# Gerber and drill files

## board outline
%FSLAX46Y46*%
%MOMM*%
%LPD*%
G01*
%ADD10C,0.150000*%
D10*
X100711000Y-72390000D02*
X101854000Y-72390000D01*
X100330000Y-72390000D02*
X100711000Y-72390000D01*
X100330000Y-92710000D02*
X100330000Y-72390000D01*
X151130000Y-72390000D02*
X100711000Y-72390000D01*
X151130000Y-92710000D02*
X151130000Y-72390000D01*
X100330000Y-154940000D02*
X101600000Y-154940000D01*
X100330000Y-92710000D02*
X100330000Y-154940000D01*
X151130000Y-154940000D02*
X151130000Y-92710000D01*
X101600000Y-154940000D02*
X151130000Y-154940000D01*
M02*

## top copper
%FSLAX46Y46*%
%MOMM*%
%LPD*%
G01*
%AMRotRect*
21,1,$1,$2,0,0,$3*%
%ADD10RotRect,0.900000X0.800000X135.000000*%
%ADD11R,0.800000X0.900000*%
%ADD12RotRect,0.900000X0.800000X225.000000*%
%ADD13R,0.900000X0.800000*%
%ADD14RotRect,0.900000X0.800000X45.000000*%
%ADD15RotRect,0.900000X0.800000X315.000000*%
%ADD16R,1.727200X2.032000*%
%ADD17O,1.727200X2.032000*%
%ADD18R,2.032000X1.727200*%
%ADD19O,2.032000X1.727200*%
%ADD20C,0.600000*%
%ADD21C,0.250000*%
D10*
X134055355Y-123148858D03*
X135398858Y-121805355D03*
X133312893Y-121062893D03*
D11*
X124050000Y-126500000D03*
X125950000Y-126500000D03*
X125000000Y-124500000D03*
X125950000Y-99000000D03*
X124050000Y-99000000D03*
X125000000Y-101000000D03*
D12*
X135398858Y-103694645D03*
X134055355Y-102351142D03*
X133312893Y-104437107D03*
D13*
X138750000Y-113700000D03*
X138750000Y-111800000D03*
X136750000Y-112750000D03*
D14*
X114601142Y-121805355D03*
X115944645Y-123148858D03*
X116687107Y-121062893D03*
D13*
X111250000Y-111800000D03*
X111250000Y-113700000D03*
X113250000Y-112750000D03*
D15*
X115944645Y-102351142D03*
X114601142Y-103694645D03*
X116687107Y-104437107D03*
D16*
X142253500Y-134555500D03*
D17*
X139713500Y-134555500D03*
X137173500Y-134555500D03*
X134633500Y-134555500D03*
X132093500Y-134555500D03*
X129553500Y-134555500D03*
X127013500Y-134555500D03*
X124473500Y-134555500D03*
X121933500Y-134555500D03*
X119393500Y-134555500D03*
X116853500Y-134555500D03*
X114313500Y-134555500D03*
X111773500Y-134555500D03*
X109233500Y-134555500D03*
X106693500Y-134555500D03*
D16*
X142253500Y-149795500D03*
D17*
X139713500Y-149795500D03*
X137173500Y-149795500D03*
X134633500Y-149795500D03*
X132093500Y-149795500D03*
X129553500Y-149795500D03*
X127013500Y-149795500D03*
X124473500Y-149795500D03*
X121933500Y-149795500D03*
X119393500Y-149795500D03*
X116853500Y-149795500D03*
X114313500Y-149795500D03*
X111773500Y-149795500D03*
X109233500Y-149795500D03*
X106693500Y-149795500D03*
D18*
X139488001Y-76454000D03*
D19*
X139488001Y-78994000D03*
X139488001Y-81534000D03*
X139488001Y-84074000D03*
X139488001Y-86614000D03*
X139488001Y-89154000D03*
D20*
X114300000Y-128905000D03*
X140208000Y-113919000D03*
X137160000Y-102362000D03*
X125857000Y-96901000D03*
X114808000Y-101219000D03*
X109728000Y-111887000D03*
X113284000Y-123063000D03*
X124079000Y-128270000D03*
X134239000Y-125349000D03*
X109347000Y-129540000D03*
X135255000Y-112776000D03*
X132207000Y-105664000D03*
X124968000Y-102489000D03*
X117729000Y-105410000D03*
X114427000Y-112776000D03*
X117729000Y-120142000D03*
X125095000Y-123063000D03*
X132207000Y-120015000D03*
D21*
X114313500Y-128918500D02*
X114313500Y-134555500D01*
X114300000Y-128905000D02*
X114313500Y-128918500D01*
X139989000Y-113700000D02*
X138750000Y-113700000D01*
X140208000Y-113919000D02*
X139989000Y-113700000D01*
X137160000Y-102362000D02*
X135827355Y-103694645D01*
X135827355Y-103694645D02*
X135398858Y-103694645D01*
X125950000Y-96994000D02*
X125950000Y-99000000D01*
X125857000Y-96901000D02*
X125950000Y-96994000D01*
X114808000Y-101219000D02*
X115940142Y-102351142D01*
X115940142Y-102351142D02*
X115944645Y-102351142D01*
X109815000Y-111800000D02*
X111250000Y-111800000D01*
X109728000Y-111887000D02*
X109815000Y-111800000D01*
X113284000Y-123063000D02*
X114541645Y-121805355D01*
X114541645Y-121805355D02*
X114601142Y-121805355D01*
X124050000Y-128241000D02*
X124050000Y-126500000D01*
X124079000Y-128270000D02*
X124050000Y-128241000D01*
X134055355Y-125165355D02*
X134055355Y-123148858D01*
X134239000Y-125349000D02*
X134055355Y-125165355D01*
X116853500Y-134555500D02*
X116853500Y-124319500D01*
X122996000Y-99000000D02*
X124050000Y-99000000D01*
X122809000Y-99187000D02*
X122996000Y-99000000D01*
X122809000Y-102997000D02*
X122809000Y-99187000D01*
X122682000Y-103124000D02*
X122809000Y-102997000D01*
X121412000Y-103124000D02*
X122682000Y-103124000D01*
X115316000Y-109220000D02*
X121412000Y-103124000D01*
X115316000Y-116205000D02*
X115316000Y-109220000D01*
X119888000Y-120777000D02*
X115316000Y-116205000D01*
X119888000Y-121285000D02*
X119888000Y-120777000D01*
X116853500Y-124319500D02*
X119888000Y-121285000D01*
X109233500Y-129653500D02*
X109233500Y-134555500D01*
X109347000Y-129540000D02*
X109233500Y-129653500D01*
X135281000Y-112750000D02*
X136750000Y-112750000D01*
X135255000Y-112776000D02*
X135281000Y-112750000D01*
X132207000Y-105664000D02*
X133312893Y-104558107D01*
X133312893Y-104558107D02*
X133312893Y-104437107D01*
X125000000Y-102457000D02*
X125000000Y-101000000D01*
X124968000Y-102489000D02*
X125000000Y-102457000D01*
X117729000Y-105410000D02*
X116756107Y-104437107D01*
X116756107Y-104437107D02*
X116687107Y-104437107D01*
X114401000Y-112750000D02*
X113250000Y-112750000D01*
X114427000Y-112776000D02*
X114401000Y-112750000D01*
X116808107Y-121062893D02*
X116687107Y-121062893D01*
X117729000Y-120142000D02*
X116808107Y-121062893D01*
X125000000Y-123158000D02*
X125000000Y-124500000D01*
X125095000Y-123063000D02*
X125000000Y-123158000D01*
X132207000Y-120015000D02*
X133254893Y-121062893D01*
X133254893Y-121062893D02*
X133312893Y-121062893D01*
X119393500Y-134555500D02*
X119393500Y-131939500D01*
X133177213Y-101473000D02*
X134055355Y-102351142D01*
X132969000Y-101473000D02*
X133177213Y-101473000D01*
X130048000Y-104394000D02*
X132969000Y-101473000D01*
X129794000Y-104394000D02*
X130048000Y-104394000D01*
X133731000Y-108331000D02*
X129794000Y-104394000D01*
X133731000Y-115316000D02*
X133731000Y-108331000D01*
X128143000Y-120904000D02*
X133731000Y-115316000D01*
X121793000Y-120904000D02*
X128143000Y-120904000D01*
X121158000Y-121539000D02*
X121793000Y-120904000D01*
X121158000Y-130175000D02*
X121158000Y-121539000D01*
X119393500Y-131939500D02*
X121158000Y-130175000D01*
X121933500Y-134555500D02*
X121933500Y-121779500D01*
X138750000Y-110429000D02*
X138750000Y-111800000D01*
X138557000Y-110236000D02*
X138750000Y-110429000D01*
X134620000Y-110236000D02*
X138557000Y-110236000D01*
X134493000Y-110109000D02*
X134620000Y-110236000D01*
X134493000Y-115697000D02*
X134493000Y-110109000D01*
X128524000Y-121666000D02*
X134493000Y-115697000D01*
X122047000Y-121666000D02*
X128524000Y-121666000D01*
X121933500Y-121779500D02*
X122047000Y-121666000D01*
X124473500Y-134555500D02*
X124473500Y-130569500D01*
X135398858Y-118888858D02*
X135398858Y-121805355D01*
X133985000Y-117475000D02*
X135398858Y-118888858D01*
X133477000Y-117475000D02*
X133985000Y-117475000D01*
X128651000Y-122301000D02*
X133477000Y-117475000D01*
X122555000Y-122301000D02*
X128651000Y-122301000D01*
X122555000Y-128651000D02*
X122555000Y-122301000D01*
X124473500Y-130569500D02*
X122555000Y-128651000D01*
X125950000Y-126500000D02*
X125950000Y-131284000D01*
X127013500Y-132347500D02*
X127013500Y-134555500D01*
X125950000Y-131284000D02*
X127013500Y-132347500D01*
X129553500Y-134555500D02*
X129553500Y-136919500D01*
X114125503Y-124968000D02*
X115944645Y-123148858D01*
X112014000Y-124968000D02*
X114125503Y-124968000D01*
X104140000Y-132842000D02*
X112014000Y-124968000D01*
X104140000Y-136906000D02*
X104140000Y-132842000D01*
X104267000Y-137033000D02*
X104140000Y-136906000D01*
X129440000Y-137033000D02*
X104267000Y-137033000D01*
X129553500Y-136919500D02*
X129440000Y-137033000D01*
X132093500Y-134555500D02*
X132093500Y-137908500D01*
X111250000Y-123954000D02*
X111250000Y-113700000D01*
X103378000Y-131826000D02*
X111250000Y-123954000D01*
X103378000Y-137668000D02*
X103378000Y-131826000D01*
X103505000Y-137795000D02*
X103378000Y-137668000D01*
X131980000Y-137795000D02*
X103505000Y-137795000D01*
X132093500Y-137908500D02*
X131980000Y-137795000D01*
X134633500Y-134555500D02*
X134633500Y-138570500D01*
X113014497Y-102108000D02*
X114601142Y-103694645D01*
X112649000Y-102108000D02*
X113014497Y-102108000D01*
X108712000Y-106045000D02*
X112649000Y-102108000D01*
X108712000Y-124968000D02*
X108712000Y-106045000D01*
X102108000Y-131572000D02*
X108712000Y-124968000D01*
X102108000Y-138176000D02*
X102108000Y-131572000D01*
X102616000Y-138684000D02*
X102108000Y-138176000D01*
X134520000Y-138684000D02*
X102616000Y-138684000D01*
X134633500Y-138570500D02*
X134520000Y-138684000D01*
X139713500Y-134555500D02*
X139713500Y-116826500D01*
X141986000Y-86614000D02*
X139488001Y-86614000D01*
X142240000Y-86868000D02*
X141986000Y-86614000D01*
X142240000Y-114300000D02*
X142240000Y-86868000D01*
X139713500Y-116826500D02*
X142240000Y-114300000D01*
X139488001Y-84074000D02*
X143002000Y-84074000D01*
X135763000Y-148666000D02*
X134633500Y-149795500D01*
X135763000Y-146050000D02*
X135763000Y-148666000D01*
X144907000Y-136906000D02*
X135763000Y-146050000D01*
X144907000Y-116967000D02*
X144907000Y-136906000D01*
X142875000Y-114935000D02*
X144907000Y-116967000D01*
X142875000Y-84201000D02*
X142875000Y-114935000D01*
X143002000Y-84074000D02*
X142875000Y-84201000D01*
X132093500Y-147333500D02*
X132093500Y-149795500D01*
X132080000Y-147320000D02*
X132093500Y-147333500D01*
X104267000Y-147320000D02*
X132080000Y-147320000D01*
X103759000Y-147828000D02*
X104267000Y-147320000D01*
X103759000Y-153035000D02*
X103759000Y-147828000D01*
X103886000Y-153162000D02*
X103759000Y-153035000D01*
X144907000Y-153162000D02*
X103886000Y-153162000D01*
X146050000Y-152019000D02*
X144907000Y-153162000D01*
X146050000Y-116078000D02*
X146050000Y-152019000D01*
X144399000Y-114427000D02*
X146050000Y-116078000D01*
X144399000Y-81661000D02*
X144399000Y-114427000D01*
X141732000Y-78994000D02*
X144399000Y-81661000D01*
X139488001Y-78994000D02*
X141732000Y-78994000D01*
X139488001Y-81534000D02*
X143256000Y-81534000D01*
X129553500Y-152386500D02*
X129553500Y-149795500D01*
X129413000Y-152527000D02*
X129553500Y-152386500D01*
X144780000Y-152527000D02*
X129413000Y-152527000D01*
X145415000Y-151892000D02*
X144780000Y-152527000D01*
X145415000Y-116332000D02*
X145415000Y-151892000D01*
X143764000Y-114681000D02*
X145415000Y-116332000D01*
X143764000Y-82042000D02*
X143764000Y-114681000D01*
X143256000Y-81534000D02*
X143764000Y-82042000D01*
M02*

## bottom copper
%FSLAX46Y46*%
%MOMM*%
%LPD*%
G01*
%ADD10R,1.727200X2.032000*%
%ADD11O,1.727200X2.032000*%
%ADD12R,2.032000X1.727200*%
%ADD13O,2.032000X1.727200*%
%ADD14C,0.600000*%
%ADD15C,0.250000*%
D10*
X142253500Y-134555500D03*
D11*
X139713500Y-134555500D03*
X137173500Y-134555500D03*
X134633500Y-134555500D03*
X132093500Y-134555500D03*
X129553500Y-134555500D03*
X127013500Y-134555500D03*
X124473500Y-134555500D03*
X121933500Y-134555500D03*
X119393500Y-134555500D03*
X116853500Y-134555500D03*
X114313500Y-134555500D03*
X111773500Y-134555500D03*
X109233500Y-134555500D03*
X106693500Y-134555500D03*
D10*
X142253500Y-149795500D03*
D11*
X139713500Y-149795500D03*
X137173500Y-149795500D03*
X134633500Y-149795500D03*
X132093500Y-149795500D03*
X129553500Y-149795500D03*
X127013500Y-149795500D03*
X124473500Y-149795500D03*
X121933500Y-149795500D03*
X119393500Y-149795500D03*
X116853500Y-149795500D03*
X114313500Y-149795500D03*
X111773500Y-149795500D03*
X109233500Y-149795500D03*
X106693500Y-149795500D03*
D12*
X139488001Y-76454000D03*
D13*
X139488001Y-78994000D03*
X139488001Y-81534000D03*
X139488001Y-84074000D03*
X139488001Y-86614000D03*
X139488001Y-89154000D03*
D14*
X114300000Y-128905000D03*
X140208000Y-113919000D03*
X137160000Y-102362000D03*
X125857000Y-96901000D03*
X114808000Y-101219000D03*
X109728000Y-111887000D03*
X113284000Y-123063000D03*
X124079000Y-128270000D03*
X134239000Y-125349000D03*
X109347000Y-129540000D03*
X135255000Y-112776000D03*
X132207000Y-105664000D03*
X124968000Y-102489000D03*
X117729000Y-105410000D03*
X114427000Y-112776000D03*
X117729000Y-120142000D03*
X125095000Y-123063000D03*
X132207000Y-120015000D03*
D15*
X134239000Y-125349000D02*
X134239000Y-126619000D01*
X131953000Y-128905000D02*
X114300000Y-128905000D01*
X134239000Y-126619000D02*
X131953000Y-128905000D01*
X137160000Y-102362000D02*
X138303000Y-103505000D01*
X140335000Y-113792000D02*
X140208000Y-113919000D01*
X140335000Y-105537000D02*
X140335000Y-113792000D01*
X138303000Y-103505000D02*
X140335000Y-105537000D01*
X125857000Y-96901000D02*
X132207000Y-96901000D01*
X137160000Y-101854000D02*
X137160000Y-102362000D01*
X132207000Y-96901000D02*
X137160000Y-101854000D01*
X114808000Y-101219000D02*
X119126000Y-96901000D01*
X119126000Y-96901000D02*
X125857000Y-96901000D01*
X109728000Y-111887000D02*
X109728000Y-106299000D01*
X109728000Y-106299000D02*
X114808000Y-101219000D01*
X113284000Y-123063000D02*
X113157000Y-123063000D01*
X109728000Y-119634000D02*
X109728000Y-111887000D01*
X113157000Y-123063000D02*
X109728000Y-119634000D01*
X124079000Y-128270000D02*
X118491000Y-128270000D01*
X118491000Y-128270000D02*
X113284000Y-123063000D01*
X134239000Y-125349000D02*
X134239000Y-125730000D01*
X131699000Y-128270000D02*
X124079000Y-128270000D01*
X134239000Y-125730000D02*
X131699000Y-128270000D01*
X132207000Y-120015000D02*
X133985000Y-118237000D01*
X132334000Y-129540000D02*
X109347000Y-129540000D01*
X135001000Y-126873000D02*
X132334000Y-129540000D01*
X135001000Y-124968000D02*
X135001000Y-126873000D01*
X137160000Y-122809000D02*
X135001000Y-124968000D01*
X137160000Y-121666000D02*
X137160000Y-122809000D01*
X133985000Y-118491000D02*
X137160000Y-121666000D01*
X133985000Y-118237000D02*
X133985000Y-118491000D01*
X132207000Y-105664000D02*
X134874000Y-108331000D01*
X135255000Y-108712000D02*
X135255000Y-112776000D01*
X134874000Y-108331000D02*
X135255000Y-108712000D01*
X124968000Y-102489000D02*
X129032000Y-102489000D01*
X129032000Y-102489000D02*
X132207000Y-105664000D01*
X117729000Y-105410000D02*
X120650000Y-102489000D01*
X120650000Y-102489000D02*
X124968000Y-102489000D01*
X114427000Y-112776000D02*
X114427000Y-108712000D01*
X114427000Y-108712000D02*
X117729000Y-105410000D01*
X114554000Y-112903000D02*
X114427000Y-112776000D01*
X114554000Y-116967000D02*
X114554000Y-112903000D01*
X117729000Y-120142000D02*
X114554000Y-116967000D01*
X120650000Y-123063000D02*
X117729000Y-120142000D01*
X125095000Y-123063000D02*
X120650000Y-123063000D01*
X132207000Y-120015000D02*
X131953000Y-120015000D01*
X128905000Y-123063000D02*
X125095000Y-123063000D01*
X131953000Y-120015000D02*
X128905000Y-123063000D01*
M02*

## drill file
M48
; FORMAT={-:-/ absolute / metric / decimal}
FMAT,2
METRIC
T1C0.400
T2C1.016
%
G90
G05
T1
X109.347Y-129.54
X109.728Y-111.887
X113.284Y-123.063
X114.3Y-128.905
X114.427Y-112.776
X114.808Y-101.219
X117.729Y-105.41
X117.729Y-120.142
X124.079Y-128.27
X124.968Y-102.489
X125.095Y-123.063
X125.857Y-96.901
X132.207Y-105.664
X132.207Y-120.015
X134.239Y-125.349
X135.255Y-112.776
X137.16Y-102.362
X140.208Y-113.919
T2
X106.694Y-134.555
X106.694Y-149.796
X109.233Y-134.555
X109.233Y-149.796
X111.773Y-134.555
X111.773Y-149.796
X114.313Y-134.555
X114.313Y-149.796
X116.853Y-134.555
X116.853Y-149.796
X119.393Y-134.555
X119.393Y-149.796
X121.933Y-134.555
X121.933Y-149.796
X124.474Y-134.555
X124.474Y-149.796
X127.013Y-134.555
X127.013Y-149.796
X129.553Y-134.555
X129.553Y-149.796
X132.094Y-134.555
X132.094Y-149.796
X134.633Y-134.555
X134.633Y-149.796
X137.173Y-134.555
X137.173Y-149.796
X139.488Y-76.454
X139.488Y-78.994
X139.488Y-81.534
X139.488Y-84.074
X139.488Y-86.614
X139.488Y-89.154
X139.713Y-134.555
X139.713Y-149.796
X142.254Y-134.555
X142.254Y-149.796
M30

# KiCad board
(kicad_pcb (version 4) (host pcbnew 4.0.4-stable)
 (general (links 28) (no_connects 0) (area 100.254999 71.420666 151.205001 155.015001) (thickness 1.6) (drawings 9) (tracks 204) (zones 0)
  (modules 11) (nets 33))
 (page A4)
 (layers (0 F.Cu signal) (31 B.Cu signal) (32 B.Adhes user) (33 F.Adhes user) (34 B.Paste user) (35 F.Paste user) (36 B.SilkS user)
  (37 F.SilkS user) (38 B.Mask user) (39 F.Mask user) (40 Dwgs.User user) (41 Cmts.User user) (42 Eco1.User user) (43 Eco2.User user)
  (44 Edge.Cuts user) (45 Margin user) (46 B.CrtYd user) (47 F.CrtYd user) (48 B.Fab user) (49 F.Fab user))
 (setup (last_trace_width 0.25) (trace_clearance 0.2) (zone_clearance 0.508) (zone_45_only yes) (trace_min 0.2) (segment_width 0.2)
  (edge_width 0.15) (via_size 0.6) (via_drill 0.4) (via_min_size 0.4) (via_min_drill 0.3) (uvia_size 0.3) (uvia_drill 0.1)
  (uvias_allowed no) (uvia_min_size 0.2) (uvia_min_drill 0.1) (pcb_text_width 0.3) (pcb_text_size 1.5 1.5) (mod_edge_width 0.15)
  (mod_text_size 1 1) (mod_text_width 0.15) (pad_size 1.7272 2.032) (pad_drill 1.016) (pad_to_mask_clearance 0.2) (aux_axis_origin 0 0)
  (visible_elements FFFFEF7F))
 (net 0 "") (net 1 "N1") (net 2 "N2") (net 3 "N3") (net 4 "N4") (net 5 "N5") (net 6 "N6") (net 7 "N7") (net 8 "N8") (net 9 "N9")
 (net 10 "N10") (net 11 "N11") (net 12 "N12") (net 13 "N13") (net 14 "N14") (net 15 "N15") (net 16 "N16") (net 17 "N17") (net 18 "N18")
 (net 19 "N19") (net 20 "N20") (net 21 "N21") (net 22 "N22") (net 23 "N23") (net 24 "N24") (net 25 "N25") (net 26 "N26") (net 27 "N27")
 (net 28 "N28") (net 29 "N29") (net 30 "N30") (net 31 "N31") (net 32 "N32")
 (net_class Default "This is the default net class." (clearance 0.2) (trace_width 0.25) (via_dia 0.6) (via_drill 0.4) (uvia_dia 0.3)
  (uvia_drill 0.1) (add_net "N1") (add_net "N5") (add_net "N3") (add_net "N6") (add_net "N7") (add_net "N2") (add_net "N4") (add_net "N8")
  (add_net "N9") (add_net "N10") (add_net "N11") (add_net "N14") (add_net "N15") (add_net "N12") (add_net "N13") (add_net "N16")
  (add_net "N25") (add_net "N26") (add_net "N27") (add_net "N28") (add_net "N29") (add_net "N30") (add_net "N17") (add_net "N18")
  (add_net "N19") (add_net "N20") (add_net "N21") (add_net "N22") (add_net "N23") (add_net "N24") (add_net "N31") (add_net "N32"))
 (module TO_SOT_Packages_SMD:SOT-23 (layer F.Cu) (at 134.02 121.77 135)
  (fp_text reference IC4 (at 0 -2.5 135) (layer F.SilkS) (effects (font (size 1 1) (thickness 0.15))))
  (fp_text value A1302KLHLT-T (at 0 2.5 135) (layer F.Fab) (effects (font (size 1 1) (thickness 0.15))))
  (pad 1 smd rect (at -1 -0.95 135) (size 0.9 0.8) (layers F.Cu F.Paste F.Mask) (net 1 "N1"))
  (pad 2 smd rect (at -1 0.95 135) (size 0.9 0.8) (layers F.Cu F.Paste F.Mask) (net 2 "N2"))
  (pad 3 smd rect (at 1 0 135) (size 0.9 0.8) (layers F.Cu F.Paste F.Mask) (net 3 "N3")))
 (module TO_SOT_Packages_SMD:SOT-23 (layer F.Cu) (at 125 125.5 90)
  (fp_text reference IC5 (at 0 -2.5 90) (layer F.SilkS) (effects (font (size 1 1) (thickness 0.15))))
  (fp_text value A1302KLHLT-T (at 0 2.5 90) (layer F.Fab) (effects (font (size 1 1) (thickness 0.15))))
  (pad 1 smd rect (at -1 -0.95 90) (size 0.9 0.8) (layers F.Cu F.Paste F.Mask) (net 1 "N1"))
  (pad 2 smd rect (at -1 0.95 90) (size 0.9 0.8) (layers F.Cu F.Paste F.Mask) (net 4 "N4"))
  (pad 3 smd rect (at 1 0 90) (size 0.9 0.8) (layers F.Cu F.Paste F.Mask) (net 3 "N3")))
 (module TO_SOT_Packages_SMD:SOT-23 (layer F.Cu) (at 125 100 270)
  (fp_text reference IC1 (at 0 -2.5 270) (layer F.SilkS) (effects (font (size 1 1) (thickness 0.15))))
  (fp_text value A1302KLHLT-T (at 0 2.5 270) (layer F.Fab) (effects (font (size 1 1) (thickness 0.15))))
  (pad 1 smd rect (at -1 -0.95 270) (size 0.9 0.8) (layers F.Cu F.Paste F.Mask) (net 1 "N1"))
  (pad 2 smd rect (at -1 0.95 270) (size 0.9 0.8) (layers F.Cu F.Paste F.Mask) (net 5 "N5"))
  (pad 3 smd rect (at 1 0 270) (size 0.9 0.8) (layers F.Cu F.Paste F.Mask) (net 3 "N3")))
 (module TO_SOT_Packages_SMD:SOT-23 (layer F.Cu) (at 134.02 103.73 225)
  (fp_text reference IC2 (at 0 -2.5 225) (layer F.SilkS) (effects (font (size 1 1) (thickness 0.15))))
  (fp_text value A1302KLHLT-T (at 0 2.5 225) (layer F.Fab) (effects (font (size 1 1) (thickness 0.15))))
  (pad 1 smd rect (at -1 -0.95 225) (size 0.9 0.8) (layers F.Cu F.Paste F.Mask) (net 1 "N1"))
  (pad 2 smd rect (at -1 0.95 225) (size 0.9 0.8) (layers F.Cu F.Paste F.Mask) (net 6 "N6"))
  (pad 3 smd rect (at 1 0 225) (size 0.9 0.8) (layers F.Cu F.Paste F.Mask) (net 3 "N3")))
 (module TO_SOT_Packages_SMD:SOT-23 (layer F.Cu) (at 137.75 112.75 180)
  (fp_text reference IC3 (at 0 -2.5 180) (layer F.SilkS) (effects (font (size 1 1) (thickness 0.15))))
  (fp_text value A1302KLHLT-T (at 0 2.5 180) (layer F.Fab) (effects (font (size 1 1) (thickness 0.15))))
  (pad 1 smd rect (at -1 -0.95 180) (size 0.9 0.8) (layers F.Cu F.Paste F.Mask) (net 1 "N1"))
  (pad 2 smd rect (at -1 0.95 180) (size 0.9 0.8) (layers F.Cu F.Paste F.Mask) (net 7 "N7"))
  (pad 3 smd rect (at 1 0 180) (size 0.9 0.8) (layers F.Cu F.Paste F.Mask) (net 3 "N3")))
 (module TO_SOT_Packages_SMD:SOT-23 (layer F.Cu) (at 115.98 121.77 45)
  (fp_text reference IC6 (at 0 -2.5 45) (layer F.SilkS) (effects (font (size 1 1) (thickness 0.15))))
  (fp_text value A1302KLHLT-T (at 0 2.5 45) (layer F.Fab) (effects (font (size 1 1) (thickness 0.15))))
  (pad 1 smd rect (at -1 -0.95 45) (size 0.9 0.8) (layers F.Cu F.Paste F.Mask) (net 1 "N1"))
  (pad 2 smd rect (at -1 0.95 45) (size 0.9 0.8) (layers F.Cu F.Paste F.Mask) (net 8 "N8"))
  (pad 3 smd rect (at 1 0 45) (size 0.9 0.8) (layers F.Cu F.Paste F.Mask) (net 3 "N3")))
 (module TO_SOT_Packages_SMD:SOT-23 (layer F.Cu) (at 112.25 112.75)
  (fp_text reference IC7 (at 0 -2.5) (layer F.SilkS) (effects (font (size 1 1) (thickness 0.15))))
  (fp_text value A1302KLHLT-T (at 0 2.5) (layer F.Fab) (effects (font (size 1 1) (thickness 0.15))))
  (pad 1 smd rect (at -1 -0.95) (size 0.9 0.8) (layers F.Cu F.Paste F.Mask) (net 1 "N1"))
  (pad 2 smd rect (at -1 0.95) (size 0.9 0.8) (layers F.Cu F.Paste F.Mask) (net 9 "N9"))
  (pad 3 smd rect (at 1 0) (size 0.9 0.8) (layers F.Cu F.Paste F.Mask) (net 3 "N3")))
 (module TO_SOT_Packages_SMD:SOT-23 (layer F.Cu) (at 115.98 103.73 315)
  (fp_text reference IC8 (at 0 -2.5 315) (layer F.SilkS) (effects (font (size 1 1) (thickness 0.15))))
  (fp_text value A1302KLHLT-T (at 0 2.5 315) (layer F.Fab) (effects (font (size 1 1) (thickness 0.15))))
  (pad 1 smd rect (at -1 -0.95 315) (size 0.9 0.8) (layers F.Cu F.Paste F.Mask) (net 1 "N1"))
  (pad 2 smd rect (at -1 0.95 315) (size 0.9 0.8) (layers F.Cu F.Paste F.Mask) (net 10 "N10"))
  (pad 3 smd rect (at 1 0 315) (size 0.9 0.8) (layers F.Cu F.Paste F.Mask) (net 3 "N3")))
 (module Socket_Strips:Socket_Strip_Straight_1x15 (layer B.Cu) (at 142.2535 134.5555 180)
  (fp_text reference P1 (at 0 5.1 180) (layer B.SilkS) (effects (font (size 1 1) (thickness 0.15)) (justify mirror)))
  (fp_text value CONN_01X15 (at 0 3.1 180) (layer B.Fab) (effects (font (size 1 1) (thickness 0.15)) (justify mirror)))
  (pad 1 thru_hole rect (at 0 0 180) (size 1.7272 2.032) (drill 1.016) (layers *.Cu *.Mask) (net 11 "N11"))
  (pad 2 thru_hole oval (at 2.54 0 180) (size 1.7272 2.032) (drill 1.016) (layers *.Cu *.Mask) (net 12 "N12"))
  (pad 3 thru_hole oval (at 5.08 0 180) (size 1.7272 2.032) (drill 1.016) (layers *.Cu *.Mask) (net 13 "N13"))
  (pad 4 thru_hole oval (at 7.62 0 180) (size 1.7272 2.032) (drill 1.016) (layers *.Cu *.Mask) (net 10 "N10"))
  (pad 5 thru_hole oval (at 10.16 0 180) (size 1.7272 2.032) (drill 1.016) (layers *.Cu *.Mask) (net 9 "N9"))
  (pad 6 thru_hole oval (at 12.7 0 180) (size 1.7272 2.032) (drill 1.016) (layers *.Cu *.Mask) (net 8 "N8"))
  (pad 7 thru_hole oval (at 15.24 0 180) (size 1.7272 2.032) (drill 1.016) (layers *.Cu *.Mask) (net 4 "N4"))
  (pad 8 thru_hole oval (at 17.78 0 180) (size 1.7272 2.032) (drill 1.016) (layers *.Cu *.Mask) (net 2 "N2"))
  (pad 9 thru_hole oval (at 20.32 0 180) (size 1.7272 2.032) (drill 1.016) (layers *.Cu *.Mask) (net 7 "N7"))
  (pad 10 thru_hole oval (at 22.86 0 180) (size 1.7272 2.032) (drill 1.016) (layers *.Cu *.Mask) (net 6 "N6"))
  (pad 11 thru_hole oval (at 25.4 0 180) (size 1.7272 2.032) (drill 1.016) (layers *.Cu *.Mask) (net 5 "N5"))
  (pad 12 thru_hole oval (at 27.94 0 180) (size 1.7272 2.032) (drill 1.016) (layers *.Cu *.Mask) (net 1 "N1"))
  (pad 13 thru_hole oval (at 30.48 0 180) (size 1.7272 2.032) (drill 1.016) (layers *.Cu *.Mask) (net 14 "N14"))
  (pad 14 thru_hole oval (at 33.02 0 180) (size 1.7272 2.032) (drill 1.016) (layers *.Cu *.Mask) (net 3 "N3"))
  (pad 15 thru_hole oval (at 35.56 0 180) (size 1.7272 2.032) (drill 1.016) (layers *.Cu *.Mask) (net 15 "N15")))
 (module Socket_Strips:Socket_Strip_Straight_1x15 (layer B.Cu) (at 142.2535 149.7955 180)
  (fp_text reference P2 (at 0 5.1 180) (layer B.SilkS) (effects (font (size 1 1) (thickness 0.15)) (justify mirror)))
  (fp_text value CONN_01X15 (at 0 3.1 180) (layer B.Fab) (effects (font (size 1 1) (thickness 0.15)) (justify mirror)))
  (pad 1 thru_hole rect (at 0 0 180) (size 1.7272 2.032) (drill 1.016) (layers *.Cu *.Mask) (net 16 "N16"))
  (pad 2 thru_hole oval (at 2.54 0 180) (size 1.7272 2.032) (drill 1.016) (layers *.Cu *.Mask) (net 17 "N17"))
  (pad 3 thru_hole oval (at 5.08 0 180) (size 1.7272 2.032) (drill 1.016) (layers *.Cu *.Mask) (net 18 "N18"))
  (pad 4 thru_hole oval (at 7.62 0 180) (size 1.7272 2.032) (drill 1.016) (layers *.Cu *.Mask) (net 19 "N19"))
  (pad 5 thru_hole oval (at 10.16 0 180) (size 1.7272 2.032) (drill 1.016) (layers *.Cu *.Mask) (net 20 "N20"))
  (pad 6 thru_hole oval (at 12.7 0 180) (size 1.7272 2.032) (drill 1.016) (layers *.Cu *.Mask) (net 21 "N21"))
  (pad 7 thru_hole oval (at 15.24 0 180) (size 1.7272 2.032) (drill 1.016) (layers *.Cu *.Mask) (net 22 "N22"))
  (pad 8 thru_hole oval (at 17.78 0 180) (size 1.7272 2.032) (drill 1.016) (layers *.Cu *.Mask) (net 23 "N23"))
  (pad 9 thru_hole oval (at 20.32 0 180) (size 1.7272 2.032) (drill 1.016) (layers *.Cu *.Mask) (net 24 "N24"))
  (pad 10 thru_hole oval (at 22.86 0 180) (size 1.7272 2.032) (drill 1.016) (layers *.Cu *.Mask) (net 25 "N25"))
  (pad 11 thru_hole oval (at 25.4 0 180) (size 1.7272 2.032) (drill 1.016) (layers *.Cu *.Mask) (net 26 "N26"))
  (pad 12 thru_hole oval (at 27.94 0 180) (size 1.7272 2.032) (drill 1.016) (layers *.Cu *.Mask) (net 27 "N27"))
  (pad 13 thru_hole oval (at 30.48 0 180) (size 1.7272 2.032) (drill 1.016) (layers *.Cu *.Mask) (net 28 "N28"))
  (pad 14 thru_hole oval (at 33.02 0 180) (size 1.7272 2.032) (drill 1.016) (layers *.Cu *.Mask) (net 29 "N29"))
  (pad 15 thru_hole oval (at 35.56 0 180) (size 1.7272 2.032) (drill 1.016) (layers *.Cu *.Mask) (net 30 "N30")))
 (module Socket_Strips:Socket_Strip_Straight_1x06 (layer B.Cu) (at 139.488001 76.454 270)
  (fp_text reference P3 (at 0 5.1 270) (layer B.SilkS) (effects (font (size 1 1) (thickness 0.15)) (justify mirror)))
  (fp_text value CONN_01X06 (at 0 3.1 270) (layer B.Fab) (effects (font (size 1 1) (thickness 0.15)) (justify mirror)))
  (pad 1 thru_hole rect (at 0 0 270) (size 1.7272 2.032) (drill 1.016) (layers *.Cu *.Mask) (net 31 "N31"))
  (pad 2 thru_hole oval (at 2.54 0 270) (size 1.7272 2.032) (drill 1.016) (layers *.Cu *.Mask) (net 20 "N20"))
  (pad 3 thru_hole oval (at 5.08 0 270) (size 1.7272 2.032) (drill 1.016) (layers *.Cu *.Mask) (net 21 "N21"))
  (pad 4 thru_hole oval (at 7.62 0 270) (size 1.7272 2.032) (drill 1.016) (layers *.Cu *.Mask) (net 19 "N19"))
  (pad 5 thru_hole oval (at 10.16 0 270) (size 1.7272 2.032) (drill 1.016) (layers *.Cu *.Mask) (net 12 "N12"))
  (pad 6 thru_hole oval (at 12.7 0 270) (size 1.7272 2.032) (drill 1.016) (layers *.Cu *.Mask) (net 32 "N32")))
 (gr_line (start 100.711 72.39) (end 101.854 72.39) (angle 90) (layer Edge.Cuts) (width 0.15))
 (gr_line (start 100.33 72.39) (end 100.711 72.39) (angle 90) (layer Edge.Cuts) (width 0.15))
 (gr_line (start 100.33 92.71) (end 100.33 72.39) (angle 90) (layer Edge.Cuts) (width 0.15))
 (gr_line (start 151.13 72.39) (end 100.711 72.39) (angle 90) (layer Edge.Cuts) (width 0.15))
 (gr_line (start 151.13 92.71) (end 151.13 72.39) (angle 90) (layer Edge.Cuts) (width 0.15))
 (gr_line (start 100.33 154.94) (end 101.6 154.94) (angle 90) (layer Edge.Cuts) (width 0.15))
 (gr_line (start 100.33 92.71) (end 100.33 154.94) (angle 90) (layer Edge.Cuts) (width 0.15))
 (gr_line (start 151.13 154.94) (end 151.13 92.71) (angle 90) (layer Edge.Cuts) (width 0.15))
 (gr_line (start 101.6 154.94) (end 151.13 154.94) (angle 90) (layer Edge.Cuts) (width 0.15))
 (segment (start 134.239 125.349) (end 134.239 126.619) (width 0.25) (layer B.Cu) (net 1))
 (segment (start 114.3135 128.9185) (end 114.3135 134.5555) (width 0.25) (layer F.Cu) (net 1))
 (segment (start 114.3 128.905) (end 114.3135 128.9185) (width 0.25) (layer F.Cu) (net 1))
 (via (at 114.3 128.905) (size 0.6) (drill 0.4) (layers F.Cu B.Cu) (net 1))
 (segment (start 131.953 128.905) (end 114.3 128.905) (width 0.25) (layer B.Cu) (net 1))
 (segment (start 134.239 126.619) (end 131.953 128.905) (width 0.25) (layer B.Cu) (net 1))
 (segment (start 137.16 102.362) (end 138.303 103.505) (width 0.25) (layer B.Cu) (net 1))
 (segment (start 139.989 113.7) (end 138.75 113.7) (width 0.25) (layer F.Cu) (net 1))
 (segment (start 140.208 113.919) (end 139.989 113.7) (width 0.25) (layer F.Cu) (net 1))
 (via (at 140.208 113.919) (size 0.6) (drill 0.4) (layers F.Cu B.Cu) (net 1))
 (segment (start 140.335 113.792) (end 140.208 113.919) (width 0.25) (layer B.Cu) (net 1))
 (segment (start 140.335 105.537) (end 140.335 113.792) (width 0.25) (layer B.Cu) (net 1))
 (segment (start 138.303 103.505) (end 140.335 105.537) (width 0.25) (layer B.Cu) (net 1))
 (segment (start 125.857 96.901) (end 132.207 96.901) (width 0.25) (layer B.Cu) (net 1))
 (segment (start 137.16 102.362) (end 135.827355 103.694645) (width 0.25) (layer F.Cu) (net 1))
 (via (at 137.16 102.362) (size 0.6) (drill 0.4) (layers F.Cu B.Cu) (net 1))
 (segment (start 137.16 101.854) (end 137.16 102.362) (width 0.25) (layer B.Cu) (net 1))
 (segment (start 132.207 96.901) (end 137.16 101.854) (width 0.25) (layer B.Cu) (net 1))
 (segment (start 135.827355 103.694645) (end 135.398858 103.694645) (width 0.25) (layer F.Cu) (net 1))
 (segment (start 114.808 101.219) (end 119.126 96.901) (width 0.25) (layer B.Cu) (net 1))
 (segment (start 125.95 96.994) (end 125.95 99) (width 0.25) (layer F.Cu) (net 1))
 (segment (start 125.857 96.901) (end 125.95 96.994) (width 0.25) (layer F.Cu) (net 1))
 (via (at 125.857 96.901) (size 0.6) (drill 0.4) (layers F.Cu B.Cu) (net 1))
 (segment (start 119.126 96.901) (end 125.857 96.901) (width 0.25) (layer B.Cu) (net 1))
 (segment (start 109.728 111.887) (end 109.728 106.299) (width 0.25) (layer B.Cu) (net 1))
 (segment (start 114.808 101.219) (end 115.940142 102.351142) (width 0.25) (layer F.Cu) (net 1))
 (via (at 114.808 101.219) (size 0.6) (drill 0.4) (layers F.Cu B.Cu) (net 1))
 (segment (start 109.728 106.299) (end 114.808 101.219) (width 0.25) (layer B.Cu) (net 1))
 (segment (start 115.940142 102.351142) (end 115.944645 102.351142) (width 0.25) (layer F.Cu) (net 1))
 (segment (start 113.284 123.063) (end 113.157 123.063) (width 0.25) (layer B.Cu) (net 1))
 (segment (start 109.815 111.8) (end 111.25 111.8) (width 0.25) (layer F.Cu) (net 1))
 (segment (start 109.728 111.887) (end 109.815 111.8) (width 0.25) (layer F.Cu) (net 1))
 (via (at 109.728 111.887) (size 0.6) (drill 0.4) (layers F.Cu B.Cu) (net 1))
 (segment (start 109.728 119.634) (end 109.728 111.887) (width 0.25) (layer B.Cu) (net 1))
 (segment (start 113.157 123.063) (end 109.728 119.634) (width 0.25) (layer B.Cu) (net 1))
 (segment (start 124.079 128.27) (end 118.491 128.27) (width 0.25) (layer B.Cu) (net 1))
 (segment (start 113.284 123.063) (end 114.541645 121.805355) (width 0.25) (layer F.Cu) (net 1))
 (via (at 113.284 123.063) (size 0.6) (drill 0.4) (layers F.Cu B.Cu) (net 1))
 (segment (start 118.491 128.27) (end 113.284 123.063) (width 0.25) (layer B.Cu) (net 1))
 (segment (start 114.541645 121.805355) (end 114.601142 121.805355) (width 0.25) (layer F.Cu) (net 1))
 (segment (start 134.239 125.349) (end 134.239 125.73) (width 0.25) (layer B.Cu) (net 1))
 (segment (start 124.05 128.241) (end 124.05 126.5) (width 0.25) (layer F.Cu) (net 1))
 (segment (start 124.079 128.27) (end 124.05 128.241) (width 0.25) (layer F.Cu) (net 1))
 (via (at 124.079 128.27) (size 0.6) (drill 0.4) (layers F.Cu B.Cu) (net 1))
 (segment (start 131.699 128.27) (end 124.079 128.27) (width 0.25) (layer B.Cu) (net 1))
 (segment (start 134.239 125.73) (end 131.699 128.27) (width 0.25) (layer B.Cu) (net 1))
 (segment (start 134.055355 125.165355) (end 134.055355 123.148858) (width 0.25) (layer F.Cu) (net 1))
 (segment (start 134.239 125.349) (end 134.055355 125.165355) (width 0.25) (layer F.Cu) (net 1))
 (via (at 134.239 125.349) (size 0.6) (drill 0.4) (layers F.Cu B.Cu) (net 1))
 (segment (start 116.8535 134.5555) (end 116.8535 124.3195) (width 0.25) (layer F.Cu) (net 5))
 (segment (start 122.996 99) (end 124.05 99) (width 0.25) (layer F.Cu) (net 5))
 (segment (start 122.809 99.187) (end 122.996 99) (width 0.25) (layer F.Cu) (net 5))
 (segment (start 122.809 102.997) (end 122.809 99.187) (width 0.25) (layer F.Cu) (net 5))
 (segment (start 122.682 103.124) (end 122.809 102.997) (width 0.25) (layer F.Cu) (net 5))
 (segment (start 121.412 103.124) (end 122.682 103.124) (width 0.25) (layer F.Cu) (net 5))
 (segment (start 115.316 109.22) (end 121.412 103.124) (width 0.25) (layer F.Cu) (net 5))
 (segment (start 115.316 116.205) (end 115.316 109.22) (width 0.25) (layer F.Cu) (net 5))
 (segment (start 119.888 120.777) (end 115.316 116.205) (width 0.25) (layer F.Cu) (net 5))
 (segment (start 119.888 121.285) (end 119.888 120.777) (width 0.25) (layer F.Cu) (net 5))
 (segment (start 116.8535 124.3195) (end 119.888 121.285) (width 0.25) (layer F.Cu) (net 5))
 (segment (start 132.207 120.015) (end 133.985 118.237) (width 0.25) (layer B.Cu) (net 3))
 (segment (start 109.2335 129.6535) (end 109.2335 134.5555) (width 0.25) (layer F.Cu) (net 3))
 (segment (start 109.347 129.54) (end 109.2335 129.6535) (width 0.25) (layer F.Cu) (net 3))
 (via (at 109.347 129.54) (size 0.6) (drill 0.4) (layers F.Cu B.Cu) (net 3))
 (segment (start 132.334 129.54) (end 109.347 129.54) (width 0.25) (layer B.Cu) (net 3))
 (segment (start 135.001 126.873) (end 132.334 129.54) (width 0.25) (layer B.Cu) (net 3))
 (segment (start 135.001 124.968) (end 135.001 126.873) (width 0.25) (layer B.Cu) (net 3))
 (segment (start 137.16 122.809) (end 135.001 124.968) (width 0.25) (layer B.Cu) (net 3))
 (segment (start 137.16 121.666) (end 137.16 122.809) (width 0.25) (layer B.Cu) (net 3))
 (segment (start 133.985 118.491) (end 137.16 121.666) (width 0.25) (layer B.Cu) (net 3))
 (segment (start 133.985 118.237) (end 133.985 118.491) (width 0.25) (layer B.Cu) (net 3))
 (segment (start 132.207 105.664) (end 134.874 108.331) (width 0.25) (layer B.Cu) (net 3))
 (segment (start 135.281 112.75) (end 136.75 112.75) (width 0.25) (layer F.Cu) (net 3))
 (segment (start 135.255 112.776) (end 135.281 112.75) (width 0.25) (layer F.Cu) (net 3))
 (via (at 135.255 112.776) (size 0.6) (drill 0.4) (layers F.Cu B.Cu) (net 3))
 (segment (start 135.255 108.712) (end 135.255 112.776) (width 0.25) (layer B.Cu) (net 3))
 (segment (start 134.874 108.331) (end 135.255 108.712) (width 0.25) (layer B.Cu) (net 3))
 (segment (start 124.968 102.489) (end 129.032 102.489) (width 0.25) (layer B.Cu) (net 3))
 (segment (start 132.207 105.664) (end 133.312893 104.558107) (width 0.25) (layer F.Cu) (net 3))
 (via (at 132.207 105.664) (size 0.6) (drill 0.4) (layers F.Cu B.Cu) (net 3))
 (segment (start 129.032 102.489) (end 132.207 105.664) (width 0.25) (layer B.Cu) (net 3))
 (segment (start 133.312893 104.558107) (end 133.312893 104.437107) (width 0.25) (layer F.Cu) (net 3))
 (segment (start 117.729 105.41) (end 120.65 102.489) (width 0.25) (layer B.Cu) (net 3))
 (segment (start 125 102.457) (end 125 101) (width 0.25) (layer F.Cu) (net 3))
 (segment (start 124.968 102.489) (end 125 102.457) (width 0.25) (layer F.Cu) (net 3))
 (via (at 124.968 102.489) (size 0.6) (drill 0.4) (layers F.Cu B.Cu) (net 3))
 (segment (start 120.65 102.489) (end 124.968 102.489) (width 0.25) (layer B.Cu) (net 3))
 (segment (start 114.427 112.776) (end 114.427 108.712) (width 0.25) (layer B.Cu) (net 3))
 (segment (start 117.729 105.41) (end 116.756107 104.437107) (width 0.25) (layer F.Cu) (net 3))
 (via (at 117.729 105.41) (size 0.6) (drill 0.4) (layers F.Cu B.Cu) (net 3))
 (segment (start 114.427 108.712) (end 117.729 105.41) (width 0.25) (layer B.Cu) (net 3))
 (segment (start 116.756107 104.437107) (end 116.687107 104.437107) (width 0.25) (layer F.Cu) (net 3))
 (segment (start 114.401 112.75) (end 113.25 112.75) (width 0.25) (layer F.Cu) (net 3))
 (segment (start 114.427 112.776) (end 114.401 112.75) (width 0.25) (layer F.Cu) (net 3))
 (via (at 114.427 112.776) (size 0.6) (drill 0.4) (layers F.Cu B.Cu) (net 3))
 (segment (start 114.554 112.903) (end 114.427 112.776) (width 0.25) (layer B.Cu) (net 3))
 (segment (start 114.554 116.967) (end 114.554 112.903) (width 0.25) (layer B.Cu) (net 3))
 (segment (start 117.729 120.142) (end 114.554 116.967) (width 0.25) (layer B.Cu) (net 3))
 (segment (start 116.808107 121.062893) (end 116.687107 121.062893) (width 0.25) (layer F.Cu) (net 3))
 (segment (start 117.729 120.142) (end 116.808107 121.062893) (width 0.25) (layer F.Cu) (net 3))
 (via (at 117.729 120.142) (size 0.6) (drill 0.4) (layers F.Cu B.Cu) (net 3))
 (segment (start 120.65 123.063) (end 117.729 120.142) (width 0.25) (layer B.Cu) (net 3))
 (segment (start 125.095 123.063) (end 120.65 123.063) (width 0.25) (layer B.Cu) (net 3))
 (segment (start 132.207 120.015) (end 131.953 120.015) (width 0.25) (layer B.Cu) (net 3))
 (segment (start 125 123.158) (end 125 124.5) (width 0.25) (layer F.Cu) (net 3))
 (segment (start 125.095 123.063) (end 125 123.158) (width 0.25) (layer F.Cu) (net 3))
 (via (at 125.095 123.063) (size 0.6) (drill 0.4) (layers F.Cu B.Cu) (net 3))
 (segment (start 128.905 123.063) (end 125.095 123.063) (width 0.25) (layer B.Cu) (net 3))
 (segment (start 131.953 120.015) (end 128.905 123.063) (width 0.25) (layer B.Cu) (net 3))
 (segment (start 132.207 120.015) (end 133.254893 121.062893) (width 0.25) (layer F.Cu) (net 3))
 (via (at 132.207 120.015) (size 0.6) (drill 0.4) (layers F.Cu B.Cu) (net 3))
 (segment (start 133.254893 121.062893) (end 133.312893 121.062893) (width 0.25) (layer F.Cu) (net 3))
 (segment (start 119.3935 134.5555) (end 119.3935 131.9395) (width 0.25) (layer F.Cu) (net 6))
 (segment (start 133.177213 101.473) (end 134.055355 102.351142) (width 0.25) (layer F.Cu) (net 6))
 (segment (start 132.969 101.473) (end 133.177213 101.473) (width 0.25) (layer F.Cu) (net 6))
 (segment (start 130.048 104.394) (end 132.969 101.473) (width 0.25) (layer F.Cu) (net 6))
 (segment (start 129.794 104.394) (end 130.048 104.394) (width 0.25) (layer F.Cu) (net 6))
 (segment (start 133.731 108.331) (end 129.794 104.394) (width 0.25) (layer F.Cu) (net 6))
 (segment (start 133.731 115.316) (end 133.731 108.331) (width 0.25) (layer F.Cu) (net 6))
 (segment (start 128.143 120.904) (end 133.731 115.316) (width 0.25) (layer F.Cu) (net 6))
 (segment (start 121.793 120.904) (end 128.143 120.904) (width 0.25) (layer F.Cu) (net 6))
 (segment (start 121.158 121.539) (end 121.793 120.904) (width 0.25) (layer F.Cu) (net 6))
 (segment (start 121.158 130.175) (end 121.158 121.539) (width 0.25) (layer F.Cu) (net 6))
 (segment (start 119.3935 131.9395) (end 121.158 130.175) (width 0.25) (layer F.Cu) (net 6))
 (segment (start 121.9335 134.5555) (end 121.9335 121.7795) (width 0.25) (layer F.Cu) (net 7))
 (segment (start 138.75 110.429) (end 138.75 111.8) (width 0.25) (layer F.Cu) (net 7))
 (segment (start 138.557 110.236) (end 138.75 110.429) (width 0.25) (layer F.Cu) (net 7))
 (segment (start 134.62 110.236) (end 138.557 110.236) (width 0.25) (layer F.Cu) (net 7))
 (segment (start 134.493 110.109) (end 134.62 110.236) (width 0.25) (layer F.Cu) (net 7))
 (segment (start 134.493 115.697) (end 134.493 110.109) (width 0.25) (layer F.Cu) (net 7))
 (segment (start 128.524 121.666) (end 134.493 115.697) (width 0.25) (layer F.Cu) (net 7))
 (segment (start 122.047 121.666) (end 128.524 121.666) (width 0.25) (layer F.Cu) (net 7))
 (segment (start 121.9335 121.7795) (end 122.047 121.666) (width 0.25) (layer F.Cu) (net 7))
 (segment (start 124.4735 134.5555) (end 124.4735 130.5695) (width 0.25) (layer F.Cu) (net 2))
 (segment (start 135.398858 118.888858) (end 135.398858 121.805355) (width 0.25) (layer F.Cu) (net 2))
 (segment (start 133.985 117.475) (end 135.398858 118.888858) (width 0.25) (layer F.Cu) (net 2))
 (segment (start 133.477 117.475) (end 133.985 117.475) (width 0.25) (layer F.Cu) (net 2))
 (segment (start 128.651 122.301) (end 133.477 117.475) (width 0.25) (layer F.Cu) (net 2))
 (segment (start 122.555 122.301) (end 128.651 122.301) (width 0.25) (layer F.Cu) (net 2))
 (segment (start 122.555 128.651) (end 122.555 122.301) (width 0.25) (layer F.Cu) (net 2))
 (segment (start 124.4735 130.5695) (end 122.555 128.651) (width 0.25) (layer F.Cu) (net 2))
 (segment (start 125.95 126.5) (end 125.95 131.284) (width 0.25) (layer F.Cu) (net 4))
 (segment (start 127.0135 132.3475) (end 127.0135 134.5555) (width 0.25) (layer F.Cu) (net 4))
 (segment (start 125.95 131.284) (end 127.0135 132.3475) (width 0.25) (layer F.Cu) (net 4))
 (segment (start 129.5535 134.5555) (end 129.5535 136.9195) (width 0.25) (layer F.Cu) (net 8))
 (segment (start 114.125503 124.968) (end 115.944645 123.148858) (width 0.25) (layer F.Cu) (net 8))
 (segment (start 112.014 124.968) (end 114.125503 124.968) (width 0.25) (layer F.Cu) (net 8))
 (segment (start 104.14 132.842) (end 112.014 124.968) (width 0.25) (layer F.Cu) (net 8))
 (segment (start 104.14 136.906) (end 104.14 132.842) (width 0.25) (layer F.Cu) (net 8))
 (segment (start 104.267 137.033) (end 104.14 136.906) (width 0.25) (layer F.Cu) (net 8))
 (segment (start 129.44 137.033) (end 104.267 137.033) (width 0.25) (layer F.Cu) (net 8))
 (segment (start 129.5535 136.9195) (end 129.44 137.033) (width 0.25) (layer F.Cu) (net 8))
 (segment (start 132.0935 134.5555) (end 132.0935 137.9085) (width 0.25) (layer F.Cu) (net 9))
 (segment (start 111.25 123.954) (end 111.25 113.7) (width 0.25) (layer F.Cu) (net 9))
 (segment (start 103.378 131.826) (end 111.25 123.954) (width 0.25) (layer F.Cu) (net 9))
 (segment (start 103.378 137.668) (end 103.378 131.826) (width 0.25) (layer F.Cu) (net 9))
 (segment (start 103.505 137.795) (end 103.378 137.668) (width 0.25) (layer F.Cu) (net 9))
 (segment (start 131.98 137.795) (end 103.505 137.795) (width 0.25) (layer F.Cu) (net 9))
 (segment (start 132.0935 137.9085) (end 131.98 137.795) (width 0.25) (layer F.Cu) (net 9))
 (segment (start 134.6335 134.5555) (end 134.6335 138.5705) (width 0.25) (layer F.Cu) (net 10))
 (segment (start 113.014497 102.108) (end 114.601142 103.694645) (width 0.25) (layer F.Cu) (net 10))
 (segment (start 112.649 102.108) (end 113.014497 102.108) (width 0.25) (layer F.Cu) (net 10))
 (segment (start 108.712 106.045) (end 112.649 102.108) (width 0.25) (layer F.Cu) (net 10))
 (segment (start 108.712 124.968) (end 108.712 106.045) (width 0.25) (layer F.Cu) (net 10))
 (segment (start 102.108 131.572) (end 108.712 124.968) (width 0.25) (layer F.Cu) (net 10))
 (segment (start 102.108 138.176) (end 102.108 131.572) (width 0.25) (layer F.Cu) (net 10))
 (segment (start 102.616 138.684) (end 102.108 138.176) (width 0.25) (layer F.Cu) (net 10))
 (segment (start 134.52 138.684) (end 102.616 138.684) (width 0.25) (layer F.Cu) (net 10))
 (segment (start 134.6335 138.5705) (end 134.52 138.684) (width 0.25) (layer F.Cu) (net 10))
 (segment (start 139.7135 134.5555) (end 139.7135 116.8265) (width 0.25) (layer F.Cu) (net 12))
 (segment (start 141.986 86.614) (end 139.488001 86.614) (width 0.25) (layer F.Cu) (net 12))
 (segment (start 142.24 86.868) (end 141.986 86.614) (width 0.25) (layer F.Cu) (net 12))
 (segment (start 142.24 114.3) (end 142.24 86.868) (width 0.25) (layer F.Cu) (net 12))
 (segment (start 139.7135 116.8265) (end 142.24 114.3) (width 0.25) (layer F.Cu) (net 12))
 (segment (start 139.488001 84.074) (end 143.002 84.074) (width 0.25) (layer F.Cu) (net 19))
 (segment (start 135.763 148.666) (end 134.6335 149.7955) (width 0.25) (layer F.Cu) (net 19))
 (segment (start 135.763 146.05) (end 135.763 148.666) (width 0.25) (layer F.Cu) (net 19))
 (segment (start 144.907 136.906) (end 135.763 146.05) (width 0.25) (layer F.Cu) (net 19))
 (segment (start 144.907 116.967) (end 144.907 136.906) (width 0.25) (layer F.Cu) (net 19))
 (segment (start 142.875 114.935) (end 144.907 116.967) (width 0.25) (layer F.Cu) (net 19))
 (segment (start 142.875 84.201) (end 142.875 114.935) (width 0.25) (layer F.Cu) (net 19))
 (segment (start 143.002 84.074) (end 142.875 84.201) (width 0.25) (layer F.Cu) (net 19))
 (segment (start 132.0935 147.3335) (end 132.0935 149.7955) (width 0.25) (layer F.Cu) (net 20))
 (segment (start 132.08 147.32) (end 132.0935 147.3335) (width 0.25) (layer F.Cu) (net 20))
 (segment (start 104.267 147.32) (end 132.08 147.32) (width 0.25) (layer F.Cu) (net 20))
 (segment (start 103.759 147.828) (end 104.267 147.32) (width 0.25) (layer F.Cu) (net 20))
 (segment (start 103.759 153.035) (end 103.759 147.828) (width 0.25) (layer F.Cu) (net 20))
 (segment (start 103.886 153.162) (end 103.759 153.035) (width 0.25) (layer F.Cu) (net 20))
 (segment (start 144.907 153.162) (end 103.886 153.162) (width 0.25) (layer F.Cu) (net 20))
 (segment (start 146.05 152.019) (end 144.907 153.162) (width 0.25) (layer F.Cu) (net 20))
 (segment (start 146.05 116.078) (end 146.05 152.019) (width 0.25) (layer F.Cu) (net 20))
 (segment (start 144.399 114.427) (end 146.05 116.078) (width 0.25) (layer F.Cu) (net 20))
 (segment (start 144.399 81.661) (end 144.399 114.427) (width 0.25) (layer F.Cu) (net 20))
 (segment (start 141.732 78.994) (end 144.399 81.661) (width 0.25) (layer F.Cu) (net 20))
 (segment (start 139.488001 78.994) (end 141.732 78.994) (width 0.25) (layer F.Cu) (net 20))
 (segment (start 139.488001 81.534) (end 143.256 81.534) (width 0.25) (layer F.Cu) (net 21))
 (segment (start 129.5535 152.3865) (end 129.5535 149.7955) (width 0.25) (layer F.Cu) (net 21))
 (segment (start 129.413 152.527) (end 129.5535 152.3865) (width 0.25) (layer F.Cu) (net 21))
 (segment (start 144.78 152.527) (end 129.413 152.527) (width 0.25) (layer F.Cu) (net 21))
 (segment (start 145.415 151.892) (end 144.78 152.527) (width 0.25) (layer F.Cu) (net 21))
 (segment (start 145.415 116.332) (end 145.415 151.892) (width 0.25) (layer F.Cu) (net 21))
 (segment (start 143.764 114.681) (end 145.415 116.332) (width 0.25) (layer F.Cu) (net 21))
 (segment (start 143.764 82.042) (end 143.764 114.681) (width 0.25) (layer F.Cu) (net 21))
 (segment (start 143.256 81.534) (end 143.764 82.042) (width 0.25) (layer F.Cu) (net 21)))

